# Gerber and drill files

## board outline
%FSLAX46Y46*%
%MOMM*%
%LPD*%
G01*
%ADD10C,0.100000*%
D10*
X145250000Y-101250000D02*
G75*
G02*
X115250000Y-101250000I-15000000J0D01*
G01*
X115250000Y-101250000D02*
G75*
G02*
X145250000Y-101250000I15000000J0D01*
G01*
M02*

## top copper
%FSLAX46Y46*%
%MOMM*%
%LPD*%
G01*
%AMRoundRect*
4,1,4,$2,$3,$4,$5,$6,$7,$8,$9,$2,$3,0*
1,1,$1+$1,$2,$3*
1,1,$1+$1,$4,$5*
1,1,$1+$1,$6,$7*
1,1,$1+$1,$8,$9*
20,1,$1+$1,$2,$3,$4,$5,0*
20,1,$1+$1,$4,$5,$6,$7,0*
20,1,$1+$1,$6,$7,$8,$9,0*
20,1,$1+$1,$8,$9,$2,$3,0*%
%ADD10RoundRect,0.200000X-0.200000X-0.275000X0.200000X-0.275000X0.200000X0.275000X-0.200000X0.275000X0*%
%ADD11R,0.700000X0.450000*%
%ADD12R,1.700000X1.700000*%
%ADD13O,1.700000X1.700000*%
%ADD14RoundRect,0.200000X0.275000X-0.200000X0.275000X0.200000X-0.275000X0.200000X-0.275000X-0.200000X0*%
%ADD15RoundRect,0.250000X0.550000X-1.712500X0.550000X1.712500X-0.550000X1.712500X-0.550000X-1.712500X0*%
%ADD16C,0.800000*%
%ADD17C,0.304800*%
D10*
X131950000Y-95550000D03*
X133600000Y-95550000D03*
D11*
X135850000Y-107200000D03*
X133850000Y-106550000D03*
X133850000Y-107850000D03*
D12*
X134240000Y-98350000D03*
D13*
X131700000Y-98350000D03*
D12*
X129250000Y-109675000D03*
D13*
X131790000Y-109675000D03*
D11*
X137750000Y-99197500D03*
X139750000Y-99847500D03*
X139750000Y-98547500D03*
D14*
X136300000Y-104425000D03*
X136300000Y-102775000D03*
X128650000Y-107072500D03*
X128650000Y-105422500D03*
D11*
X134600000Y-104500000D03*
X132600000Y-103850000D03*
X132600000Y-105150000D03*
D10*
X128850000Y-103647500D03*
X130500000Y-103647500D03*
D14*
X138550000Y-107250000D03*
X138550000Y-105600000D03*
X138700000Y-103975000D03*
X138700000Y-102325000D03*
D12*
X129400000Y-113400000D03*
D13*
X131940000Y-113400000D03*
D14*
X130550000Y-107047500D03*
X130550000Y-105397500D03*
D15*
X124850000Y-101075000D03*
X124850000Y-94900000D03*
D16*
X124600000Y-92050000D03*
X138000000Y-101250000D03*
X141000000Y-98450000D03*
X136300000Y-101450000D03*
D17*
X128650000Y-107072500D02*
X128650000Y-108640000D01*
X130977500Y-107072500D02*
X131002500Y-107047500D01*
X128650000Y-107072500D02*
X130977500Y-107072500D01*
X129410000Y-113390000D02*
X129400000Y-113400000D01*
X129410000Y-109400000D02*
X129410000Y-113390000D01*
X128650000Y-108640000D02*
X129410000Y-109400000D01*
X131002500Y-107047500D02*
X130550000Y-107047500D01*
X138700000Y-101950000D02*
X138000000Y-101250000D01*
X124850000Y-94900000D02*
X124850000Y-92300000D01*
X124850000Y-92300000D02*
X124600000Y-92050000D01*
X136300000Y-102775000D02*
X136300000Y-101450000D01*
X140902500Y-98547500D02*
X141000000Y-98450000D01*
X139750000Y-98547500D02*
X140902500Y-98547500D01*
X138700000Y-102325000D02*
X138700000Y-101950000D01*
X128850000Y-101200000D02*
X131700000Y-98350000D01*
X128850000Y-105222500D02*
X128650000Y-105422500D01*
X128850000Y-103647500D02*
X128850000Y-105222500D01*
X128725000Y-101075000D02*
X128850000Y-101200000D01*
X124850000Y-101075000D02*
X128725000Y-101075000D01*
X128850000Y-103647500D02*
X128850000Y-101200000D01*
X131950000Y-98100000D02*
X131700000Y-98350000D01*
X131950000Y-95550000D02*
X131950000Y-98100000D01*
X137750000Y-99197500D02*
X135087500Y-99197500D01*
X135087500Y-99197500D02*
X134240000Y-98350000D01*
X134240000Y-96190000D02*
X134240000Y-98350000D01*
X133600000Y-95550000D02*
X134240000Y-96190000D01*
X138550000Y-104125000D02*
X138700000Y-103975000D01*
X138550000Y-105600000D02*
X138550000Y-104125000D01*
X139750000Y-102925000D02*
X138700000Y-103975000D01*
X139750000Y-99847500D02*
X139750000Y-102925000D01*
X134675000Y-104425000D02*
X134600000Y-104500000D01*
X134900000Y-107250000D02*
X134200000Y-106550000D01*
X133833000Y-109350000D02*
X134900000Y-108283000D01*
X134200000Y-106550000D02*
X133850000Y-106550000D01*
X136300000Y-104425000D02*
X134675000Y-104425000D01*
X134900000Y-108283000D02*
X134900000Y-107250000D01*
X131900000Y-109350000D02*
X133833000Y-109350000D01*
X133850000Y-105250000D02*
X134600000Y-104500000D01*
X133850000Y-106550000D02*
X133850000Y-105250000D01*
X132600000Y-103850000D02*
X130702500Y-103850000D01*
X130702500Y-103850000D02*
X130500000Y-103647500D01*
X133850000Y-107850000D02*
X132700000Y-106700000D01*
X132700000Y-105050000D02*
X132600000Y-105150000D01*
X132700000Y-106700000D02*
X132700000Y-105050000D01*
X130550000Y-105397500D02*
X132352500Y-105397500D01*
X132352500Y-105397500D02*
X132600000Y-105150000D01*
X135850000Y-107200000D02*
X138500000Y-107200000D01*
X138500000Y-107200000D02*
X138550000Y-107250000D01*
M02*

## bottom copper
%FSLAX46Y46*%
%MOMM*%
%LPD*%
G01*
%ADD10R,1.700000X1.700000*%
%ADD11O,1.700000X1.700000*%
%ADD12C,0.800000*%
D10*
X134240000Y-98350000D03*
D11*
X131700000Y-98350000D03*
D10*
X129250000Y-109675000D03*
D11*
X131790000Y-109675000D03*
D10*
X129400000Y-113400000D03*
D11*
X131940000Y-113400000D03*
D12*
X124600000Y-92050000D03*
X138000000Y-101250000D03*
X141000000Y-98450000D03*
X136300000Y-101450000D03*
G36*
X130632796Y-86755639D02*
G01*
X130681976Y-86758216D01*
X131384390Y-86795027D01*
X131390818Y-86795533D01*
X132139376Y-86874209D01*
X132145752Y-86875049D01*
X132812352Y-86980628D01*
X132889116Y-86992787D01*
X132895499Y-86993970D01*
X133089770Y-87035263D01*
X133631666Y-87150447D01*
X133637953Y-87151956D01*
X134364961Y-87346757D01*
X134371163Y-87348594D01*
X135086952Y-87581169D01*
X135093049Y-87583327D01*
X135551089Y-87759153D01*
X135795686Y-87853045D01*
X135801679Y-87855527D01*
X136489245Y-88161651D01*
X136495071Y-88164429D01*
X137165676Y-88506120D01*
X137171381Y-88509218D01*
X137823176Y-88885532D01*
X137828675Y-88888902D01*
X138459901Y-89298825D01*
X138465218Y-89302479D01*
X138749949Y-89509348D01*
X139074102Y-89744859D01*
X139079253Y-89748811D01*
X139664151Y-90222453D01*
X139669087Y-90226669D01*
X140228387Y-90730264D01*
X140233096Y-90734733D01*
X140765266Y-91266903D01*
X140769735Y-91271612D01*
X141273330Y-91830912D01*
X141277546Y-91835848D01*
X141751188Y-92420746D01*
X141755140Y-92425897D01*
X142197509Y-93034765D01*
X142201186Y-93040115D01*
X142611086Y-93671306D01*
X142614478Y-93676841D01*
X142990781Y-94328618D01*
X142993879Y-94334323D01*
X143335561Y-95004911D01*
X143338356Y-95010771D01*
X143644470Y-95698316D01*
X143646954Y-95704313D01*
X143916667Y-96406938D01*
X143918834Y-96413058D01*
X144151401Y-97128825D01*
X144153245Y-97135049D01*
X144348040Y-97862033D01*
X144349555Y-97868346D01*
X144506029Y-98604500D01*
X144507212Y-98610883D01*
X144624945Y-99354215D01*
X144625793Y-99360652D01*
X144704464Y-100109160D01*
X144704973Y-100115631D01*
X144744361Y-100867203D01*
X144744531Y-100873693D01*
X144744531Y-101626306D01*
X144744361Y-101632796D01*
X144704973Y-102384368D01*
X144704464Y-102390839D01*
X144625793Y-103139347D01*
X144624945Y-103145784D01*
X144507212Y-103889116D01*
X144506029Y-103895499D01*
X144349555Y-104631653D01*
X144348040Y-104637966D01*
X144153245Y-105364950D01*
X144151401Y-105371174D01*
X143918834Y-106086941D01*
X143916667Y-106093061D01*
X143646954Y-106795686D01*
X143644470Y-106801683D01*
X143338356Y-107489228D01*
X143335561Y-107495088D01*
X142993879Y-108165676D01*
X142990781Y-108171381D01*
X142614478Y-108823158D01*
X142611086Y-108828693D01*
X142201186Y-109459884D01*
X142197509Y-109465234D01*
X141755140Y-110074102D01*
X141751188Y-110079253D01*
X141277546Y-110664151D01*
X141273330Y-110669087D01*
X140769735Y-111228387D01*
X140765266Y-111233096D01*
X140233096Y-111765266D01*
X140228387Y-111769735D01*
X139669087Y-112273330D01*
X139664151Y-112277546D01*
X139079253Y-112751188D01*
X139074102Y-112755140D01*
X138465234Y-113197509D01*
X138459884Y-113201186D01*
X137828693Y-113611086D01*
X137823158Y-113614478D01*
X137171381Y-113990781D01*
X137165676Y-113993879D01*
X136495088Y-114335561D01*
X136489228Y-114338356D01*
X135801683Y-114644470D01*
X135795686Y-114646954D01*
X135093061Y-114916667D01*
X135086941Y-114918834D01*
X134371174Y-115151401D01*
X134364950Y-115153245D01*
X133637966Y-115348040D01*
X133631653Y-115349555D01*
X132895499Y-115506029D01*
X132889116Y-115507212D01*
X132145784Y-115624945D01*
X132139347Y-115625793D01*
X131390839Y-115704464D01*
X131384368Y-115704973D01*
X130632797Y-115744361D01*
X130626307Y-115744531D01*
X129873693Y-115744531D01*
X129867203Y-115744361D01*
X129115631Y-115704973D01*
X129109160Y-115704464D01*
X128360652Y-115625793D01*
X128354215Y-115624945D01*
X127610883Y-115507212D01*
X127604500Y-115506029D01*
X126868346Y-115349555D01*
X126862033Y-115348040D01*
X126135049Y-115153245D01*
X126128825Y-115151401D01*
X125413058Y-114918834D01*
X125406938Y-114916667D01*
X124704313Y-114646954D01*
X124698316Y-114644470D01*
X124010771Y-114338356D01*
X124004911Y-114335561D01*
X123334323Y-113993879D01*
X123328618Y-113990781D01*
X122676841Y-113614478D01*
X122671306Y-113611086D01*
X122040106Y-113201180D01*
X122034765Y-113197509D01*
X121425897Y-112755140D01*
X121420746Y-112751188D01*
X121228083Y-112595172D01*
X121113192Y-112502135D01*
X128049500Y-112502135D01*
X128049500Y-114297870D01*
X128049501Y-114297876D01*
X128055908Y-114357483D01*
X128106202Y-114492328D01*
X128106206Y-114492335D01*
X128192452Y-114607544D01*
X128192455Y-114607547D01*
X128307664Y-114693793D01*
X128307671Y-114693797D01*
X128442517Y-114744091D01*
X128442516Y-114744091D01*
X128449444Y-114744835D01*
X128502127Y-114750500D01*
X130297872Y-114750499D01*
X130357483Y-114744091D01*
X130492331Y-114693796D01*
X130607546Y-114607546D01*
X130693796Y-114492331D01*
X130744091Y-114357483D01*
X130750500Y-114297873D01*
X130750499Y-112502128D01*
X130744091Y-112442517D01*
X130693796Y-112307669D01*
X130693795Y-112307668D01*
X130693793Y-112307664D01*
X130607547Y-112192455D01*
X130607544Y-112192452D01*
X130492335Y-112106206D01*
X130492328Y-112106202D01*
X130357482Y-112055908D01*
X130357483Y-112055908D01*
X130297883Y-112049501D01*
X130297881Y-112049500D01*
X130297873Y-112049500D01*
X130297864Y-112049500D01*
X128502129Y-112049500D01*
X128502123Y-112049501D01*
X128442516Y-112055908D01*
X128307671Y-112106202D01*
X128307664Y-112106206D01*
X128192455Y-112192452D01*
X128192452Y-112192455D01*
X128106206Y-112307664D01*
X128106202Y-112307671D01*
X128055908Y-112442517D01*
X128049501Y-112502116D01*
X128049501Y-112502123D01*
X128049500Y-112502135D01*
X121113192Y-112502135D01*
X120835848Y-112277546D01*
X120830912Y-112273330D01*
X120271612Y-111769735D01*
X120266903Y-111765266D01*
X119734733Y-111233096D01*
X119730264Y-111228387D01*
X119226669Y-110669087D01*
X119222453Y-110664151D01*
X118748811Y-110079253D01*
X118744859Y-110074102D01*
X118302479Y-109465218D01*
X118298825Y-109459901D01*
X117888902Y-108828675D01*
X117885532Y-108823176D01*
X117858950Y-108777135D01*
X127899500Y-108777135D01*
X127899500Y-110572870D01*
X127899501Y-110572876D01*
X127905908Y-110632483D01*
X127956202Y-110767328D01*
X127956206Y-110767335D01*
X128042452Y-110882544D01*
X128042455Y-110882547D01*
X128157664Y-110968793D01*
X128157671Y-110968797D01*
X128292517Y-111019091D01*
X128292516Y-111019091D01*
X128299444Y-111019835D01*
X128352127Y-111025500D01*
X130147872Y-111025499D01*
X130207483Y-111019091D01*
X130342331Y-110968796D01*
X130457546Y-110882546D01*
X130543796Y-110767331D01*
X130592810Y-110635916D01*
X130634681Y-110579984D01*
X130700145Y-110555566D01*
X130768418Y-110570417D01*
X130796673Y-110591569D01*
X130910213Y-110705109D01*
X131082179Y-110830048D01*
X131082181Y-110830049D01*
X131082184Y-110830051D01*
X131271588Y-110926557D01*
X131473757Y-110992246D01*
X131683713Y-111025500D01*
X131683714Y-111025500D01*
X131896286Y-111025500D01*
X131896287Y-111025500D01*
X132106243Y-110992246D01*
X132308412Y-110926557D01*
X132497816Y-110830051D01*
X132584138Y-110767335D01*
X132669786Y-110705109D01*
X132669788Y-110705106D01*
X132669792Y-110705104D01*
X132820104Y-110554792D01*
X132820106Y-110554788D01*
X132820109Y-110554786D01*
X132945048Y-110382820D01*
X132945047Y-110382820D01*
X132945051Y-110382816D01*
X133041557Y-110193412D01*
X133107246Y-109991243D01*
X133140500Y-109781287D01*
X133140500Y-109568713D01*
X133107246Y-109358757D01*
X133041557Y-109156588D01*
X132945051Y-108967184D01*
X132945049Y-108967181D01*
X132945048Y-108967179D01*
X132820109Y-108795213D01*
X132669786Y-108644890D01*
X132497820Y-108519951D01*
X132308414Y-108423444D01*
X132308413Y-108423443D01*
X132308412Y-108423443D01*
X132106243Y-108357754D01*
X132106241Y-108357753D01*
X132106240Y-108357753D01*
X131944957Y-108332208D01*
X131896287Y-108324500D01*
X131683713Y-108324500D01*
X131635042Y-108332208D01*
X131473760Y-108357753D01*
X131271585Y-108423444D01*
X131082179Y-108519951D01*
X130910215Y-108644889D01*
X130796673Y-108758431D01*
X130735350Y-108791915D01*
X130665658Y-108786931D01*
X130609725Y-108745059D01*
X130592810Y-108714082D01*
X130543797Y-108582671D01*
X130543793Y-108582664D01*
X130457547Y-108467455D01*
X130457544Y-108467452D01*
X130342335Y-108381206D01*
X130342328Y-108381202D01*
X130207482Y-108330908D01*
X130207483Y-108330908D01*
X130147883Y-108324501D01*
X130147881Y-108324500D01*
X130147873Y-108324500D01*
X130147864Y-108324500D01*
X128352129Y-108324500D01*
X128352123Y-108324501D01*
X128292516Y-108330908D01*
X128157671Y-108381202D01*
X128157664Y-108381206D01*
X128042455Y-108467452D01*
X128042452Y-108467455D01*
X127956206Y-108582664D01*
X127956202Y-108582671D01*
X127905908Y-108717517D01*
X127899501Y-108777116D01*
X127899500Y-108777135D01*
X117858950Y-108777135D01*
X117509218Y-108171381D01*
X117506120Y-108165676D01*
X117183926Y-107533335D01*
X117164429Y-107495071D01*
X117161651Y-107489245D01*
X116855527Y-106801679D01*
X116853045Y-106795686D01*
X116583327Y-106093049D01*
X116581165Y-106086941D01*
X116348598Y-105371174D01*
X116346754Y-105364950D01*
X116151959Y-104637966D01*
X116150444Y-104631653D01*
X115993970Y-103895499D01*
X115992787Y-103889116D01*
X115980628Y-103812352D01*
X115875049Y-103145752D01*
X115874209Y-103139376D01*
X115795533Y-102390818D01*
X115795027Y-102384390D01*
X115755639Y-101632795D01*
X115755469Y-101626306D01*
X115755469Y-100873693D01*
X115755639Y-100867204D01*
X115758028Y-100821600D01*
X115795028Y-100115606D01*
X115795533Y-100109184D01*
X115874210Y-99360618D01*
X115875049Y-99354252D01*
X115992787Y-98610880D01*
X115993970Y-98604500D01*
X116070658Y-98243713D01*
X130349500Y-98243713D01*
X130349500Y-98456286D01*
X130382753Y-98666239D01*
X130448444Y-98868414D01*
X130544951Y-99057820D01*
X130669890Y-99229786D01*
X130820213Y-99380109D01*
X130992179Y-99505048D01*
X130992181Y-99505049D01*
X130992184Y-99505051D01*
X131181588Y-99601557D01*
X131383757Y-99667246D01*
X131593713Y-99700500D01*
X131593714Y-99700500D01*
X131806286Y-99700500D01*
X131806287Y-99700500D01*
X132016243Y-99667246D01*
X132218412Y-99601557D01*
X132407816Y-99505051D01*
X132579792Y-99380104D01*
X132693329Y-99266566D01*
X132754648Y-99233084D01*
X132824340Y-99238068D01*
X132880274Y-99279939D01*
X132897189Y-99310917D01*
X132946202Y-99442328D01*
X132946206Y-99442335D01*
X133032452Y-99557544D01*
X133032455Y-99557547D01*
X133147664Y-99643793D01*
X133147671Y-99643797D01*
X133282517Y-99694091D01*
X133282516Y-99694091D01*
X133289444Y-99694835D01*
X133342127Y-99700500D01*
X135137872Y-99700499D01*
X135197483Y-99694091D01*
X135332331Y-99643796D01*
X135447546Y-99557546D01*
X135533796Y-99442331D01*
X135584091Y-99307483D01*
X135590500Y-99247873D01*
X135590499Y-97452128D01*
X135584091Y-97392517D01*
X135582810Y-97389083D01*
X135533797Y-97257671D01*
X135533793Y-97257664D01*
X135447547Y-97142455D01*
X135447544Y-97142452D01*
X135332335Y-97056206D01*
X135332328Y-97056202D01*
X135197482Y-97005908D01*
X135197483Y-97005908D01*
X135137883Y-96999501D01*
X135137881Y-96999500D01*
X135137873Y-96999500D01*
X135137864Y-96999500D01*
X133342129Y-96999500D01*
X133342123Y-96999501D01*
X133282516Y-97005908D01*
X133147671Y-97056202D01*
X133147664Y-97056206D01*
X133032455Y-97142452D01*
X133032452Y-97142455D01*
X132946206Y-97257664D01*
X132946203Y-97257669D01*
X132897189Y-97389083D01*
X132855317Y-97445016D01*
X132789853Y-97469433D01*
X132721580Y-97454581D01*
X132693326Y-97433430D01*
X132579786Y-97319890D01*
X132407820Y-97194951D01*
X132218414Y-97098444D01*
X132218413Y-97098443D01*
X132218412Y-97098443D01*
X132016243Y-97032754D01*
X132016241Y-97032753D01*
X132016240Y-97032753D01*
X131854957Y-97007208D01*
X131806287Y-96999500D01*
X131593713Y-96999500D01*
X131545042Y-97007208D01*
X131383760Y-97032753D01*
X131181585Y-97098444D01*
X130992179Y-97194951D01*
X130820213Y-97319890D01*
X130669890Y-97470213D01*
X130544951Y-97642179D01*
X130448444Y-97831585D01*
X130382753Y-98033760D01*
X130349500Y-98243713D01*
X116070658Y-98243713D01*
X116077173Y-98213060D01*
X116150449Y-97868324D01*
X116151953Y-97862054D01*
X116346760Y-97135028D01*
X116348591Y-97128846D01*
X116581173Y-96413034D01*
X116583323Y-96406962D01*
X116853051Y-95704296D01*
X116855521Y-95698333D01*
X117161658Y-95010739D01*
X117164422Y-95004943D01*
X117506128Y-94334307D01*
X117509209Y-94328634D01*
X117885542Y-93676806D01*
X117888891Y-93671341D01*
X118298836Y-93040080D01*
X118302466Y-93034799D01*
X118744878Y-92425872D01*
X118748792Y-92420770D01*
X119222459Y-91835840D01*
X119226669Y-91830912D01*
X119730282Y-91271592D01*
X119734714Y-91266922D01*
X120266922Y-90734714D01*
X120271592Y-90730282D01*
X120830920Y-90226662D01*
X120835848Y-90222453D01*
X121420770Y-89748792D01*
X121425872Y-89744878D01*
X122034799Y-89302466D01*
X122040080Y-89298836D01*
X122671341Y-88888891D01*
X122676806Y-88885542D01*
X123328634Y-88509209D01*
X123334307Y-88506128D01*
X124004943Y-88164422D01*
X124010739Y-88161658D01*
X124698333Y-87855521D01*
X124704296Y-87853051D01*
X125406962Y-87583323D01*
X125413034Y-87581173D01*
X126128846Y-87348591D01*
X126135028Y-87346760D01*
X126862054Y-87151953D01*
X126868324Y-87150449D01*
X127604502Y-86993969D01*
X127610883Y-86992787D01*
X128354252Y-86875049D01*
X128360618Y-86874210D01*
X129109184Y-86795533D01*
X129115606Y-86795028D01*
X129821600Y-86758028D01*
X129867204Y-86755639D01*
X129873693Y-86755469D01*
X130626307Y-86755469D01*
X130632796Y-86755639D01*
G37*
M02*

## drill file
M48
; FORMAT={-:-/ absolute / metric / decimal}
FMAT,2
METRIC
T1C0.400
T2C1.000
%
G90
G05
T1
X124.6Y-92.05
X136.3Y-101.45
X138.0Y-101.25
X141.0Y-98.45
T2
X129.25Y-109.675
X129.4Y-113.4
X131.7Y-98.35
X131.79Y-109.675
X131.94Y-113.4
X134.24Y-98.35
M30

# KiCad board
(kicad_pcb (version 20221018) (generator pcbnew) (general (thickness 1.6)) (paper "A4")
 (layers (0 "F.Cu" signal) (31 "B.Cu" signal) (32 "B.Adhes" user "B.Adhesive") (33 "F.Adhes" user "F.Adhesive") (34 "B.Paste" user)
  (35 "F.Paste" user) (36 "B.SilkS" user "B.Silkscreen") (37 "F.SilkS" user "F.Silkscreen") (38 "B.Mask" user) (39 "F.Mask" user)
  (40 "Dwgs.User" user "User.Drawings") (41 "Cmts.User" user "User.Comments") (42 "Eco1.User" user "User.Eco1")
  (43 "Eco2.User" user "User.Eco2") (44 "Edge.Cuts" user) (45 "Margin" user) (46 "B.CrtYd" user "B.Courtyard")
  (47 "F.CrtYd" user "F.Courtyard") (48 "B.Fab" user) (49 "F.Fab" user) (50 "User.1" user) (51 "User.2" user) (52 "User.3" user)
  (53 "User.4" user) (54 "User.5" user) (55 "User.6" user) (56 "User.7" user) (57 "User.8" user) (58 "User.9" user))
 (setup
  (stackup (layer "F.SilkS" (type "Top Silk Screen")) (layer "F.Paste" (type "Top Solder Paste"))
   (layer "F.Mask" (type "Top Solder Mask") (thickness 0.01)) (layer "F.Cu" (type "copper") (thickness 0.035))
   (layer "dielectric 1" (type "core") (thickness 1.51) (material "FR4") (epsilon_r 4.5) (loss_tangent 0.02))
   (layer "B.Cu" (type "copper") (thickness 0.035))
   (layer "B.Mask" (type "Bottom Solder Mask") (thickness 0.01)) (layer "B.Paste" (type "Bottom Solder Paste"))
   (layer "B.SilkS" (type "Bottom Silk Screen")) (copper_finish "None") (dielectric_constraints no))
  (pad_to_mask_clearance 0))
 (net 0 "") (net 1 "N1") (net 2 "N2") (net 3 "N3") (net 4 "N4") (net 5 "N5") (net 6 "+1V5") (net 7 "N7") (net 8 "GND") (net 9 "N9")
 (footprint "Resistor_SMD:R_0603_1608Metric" (layer "F.Cu") (at 132.775 95.55)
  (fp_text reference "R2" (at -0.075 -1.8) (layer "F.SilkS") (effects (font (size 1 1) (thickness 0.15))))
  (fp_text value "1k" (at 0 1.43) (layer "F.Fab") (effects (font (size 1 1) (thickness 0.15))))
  (pad "1" smd roundrect (at -0.825 0) (size 0.8 0.95) (layers "F.Cu" "F.Paste" "F.Mask") (roundrect_rratio 0.25) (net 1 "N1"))
  (pad "2" smd roundrect (at 0.825 0) (size 0.8 0.95) (layers "F.Cu" "F.Paste" "F.Mask") (roundrect_rratio 0.25) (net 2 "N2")))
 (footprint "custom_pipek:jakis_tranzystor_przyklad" (layer "F.Cu") (at 134.55 105.92)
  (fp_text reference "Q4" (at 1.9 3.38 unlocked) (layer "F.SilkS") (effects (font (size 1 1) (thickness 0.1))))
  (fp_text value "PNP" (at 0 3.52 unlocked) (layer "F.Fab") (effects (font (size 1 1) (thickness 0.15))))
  (pad "1" smd rect (at 1.3 1.28 270) (size 0.45 0.7) (layers "F.Cu" "F.Paste" "F.Mask") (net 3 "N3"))
  (pad "2" smd rect (at -0.7 0.63 270) (size 0.45 0.7) (layers "F.Cu" "F.Paste" "F.Mask") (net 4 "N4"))
  (pad "3" smd rect (at -0.7 1.93 270) (size 0.45 0.7) (layers "F.Cu" "F.Paste" "F.Mask") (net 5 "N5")))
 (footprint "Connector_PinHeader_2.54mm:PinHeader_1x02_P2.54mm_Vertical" (layer "F.Cu") (at 134.24 98.35 -90)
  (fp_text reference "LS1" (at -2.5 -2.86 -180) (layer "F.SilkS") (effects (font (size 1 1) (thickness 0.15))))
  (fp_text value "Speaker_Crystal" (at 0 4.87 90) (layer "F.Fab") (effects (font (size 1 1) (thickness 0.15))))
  (pad "1" thru_hole rect (at 0 0 270) (size 1.7 1.7) (drill 1) (layers "*.Cu" "*.Mask") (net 2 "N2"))
  (pad "2" thru_hole oval (at 0 2.54 270) (size 1.7 1.7) (drill 1) (layers "*.Cu" "*.Mask") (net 1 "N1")))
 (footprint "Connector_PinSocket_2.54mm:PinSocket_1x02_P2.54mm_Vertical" (layer "F.Cu") (at 129.25 109.675 90)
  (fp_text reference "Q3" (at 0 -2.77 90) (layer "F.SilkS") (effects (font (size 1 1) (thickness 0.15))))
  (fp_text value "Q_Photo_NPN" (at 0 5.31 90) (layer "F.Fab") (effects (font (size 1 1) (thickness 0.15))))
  (pad "1" thru_hole rect (at 0 0 90) (size 1.7 1.7) (drill 1) (layers "*.Cu" "*.Mask") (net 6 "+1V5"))
  (pad "2" thru_hole oval (at 0 2.54 90) (size 1.7 1.7) (drill 1) (layers "*.Cu" "*.Mask") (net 4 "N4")))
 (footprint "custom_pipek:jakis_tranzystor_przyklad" (layer "F.Cu") (at 139.05 100.4775 180)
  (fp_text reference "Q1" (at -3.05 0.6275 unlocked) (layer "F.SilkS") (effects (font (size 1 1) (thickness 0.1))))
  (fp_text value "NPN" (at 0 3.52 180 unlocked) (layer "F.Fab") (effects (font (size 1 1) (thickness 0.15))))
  (pad "1" smd rect (at 1.3 1.28 90) (size 0.45 0.7) (layers "F.Cu" "F.Paste" "F.Mask") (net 2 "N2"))
  (pad "2" smd rect (at -0.7 0.63 90) (size 0.45 0.7) (layers "F.Cu" "F.Paste" "F.Mask") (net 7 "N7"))
  (pad "3" smd rect (at -0.7 1.93 90) (size 0.45 0.7) (layers "F.Cu" "F.Paste" "F.Mask") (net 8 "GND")))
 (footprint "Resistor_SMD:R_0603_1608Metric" (layer "F.Cu") (at 136.3 103.6 90)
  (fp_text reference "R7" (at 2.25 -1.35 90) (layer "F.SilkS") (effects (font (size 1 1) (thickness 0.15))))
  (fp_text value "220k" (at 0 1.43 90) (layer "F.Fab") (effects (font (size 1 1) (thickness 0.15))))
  (pad "1" smd roundrect (at -0.825 0 90) (size 0.8 0.95) (layers "F.Cu" "F.Paste" "F.Mask") (roundrect_rratio 0.25) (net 4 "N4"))
  (pad "2" smd roundrect (at 0.825 0 90) (size 0.8 0.95) (layers "F.Cu" "F.Paste" "F.Mask") (roundrect_rratio 0.25) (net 8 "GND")))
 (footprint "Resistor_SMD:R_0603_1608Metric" (layer "F.Cu") (at 128.65 106.2475 90)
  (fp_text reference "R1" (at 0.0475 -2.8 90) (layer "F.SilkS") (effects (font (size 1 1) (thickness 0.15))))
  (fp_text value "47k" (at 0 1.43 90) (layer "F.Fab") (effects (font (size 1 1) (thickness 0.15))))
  (pad "1" smd roundrect (at -0.825 0 90) (size 0.8 0.95) (layers "F.Cu" "F.Paste" "F.Mask") (roundrect_rratio 0.25) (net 6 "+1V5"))
  (pad "2" smd roundrect (at 0.825 0 90) (size 0.8 0.95) (layers "F.Cu" "F.Paste" "F.Mask") (roundrect_rratio 0.25) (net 1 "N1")))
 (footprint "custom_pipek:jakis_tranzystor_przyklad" (layer "F.Cu") (at 133.3 103.22)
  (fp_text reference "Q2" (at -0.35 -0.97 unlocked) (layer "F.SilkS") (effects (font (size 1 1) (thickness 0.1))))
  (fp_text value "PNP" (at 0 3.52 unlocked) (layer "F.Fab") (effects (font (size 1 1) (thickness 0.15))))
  (pad "1" smd rect (at 1.3 1.28 270) (size 0.45 0.7) (layers "F.Cu" "F.Paste" "F.Mask") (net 4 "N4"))
  (pad "2" smd rect (at -0.7 0.63 270) (size 0.45 0.7) (layers "F.Cu" "F.Paste" "F.Mask") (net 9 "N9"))
  (pad "3" smd rect (at -0.7 1.93 270) (size 0.45 0.7) (layers "F.Cu" "F.Paste" "F.Mask") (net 5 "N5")))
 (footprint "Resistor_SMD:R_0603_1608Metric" (layer "F.Cu") (at 129.675 103.6475)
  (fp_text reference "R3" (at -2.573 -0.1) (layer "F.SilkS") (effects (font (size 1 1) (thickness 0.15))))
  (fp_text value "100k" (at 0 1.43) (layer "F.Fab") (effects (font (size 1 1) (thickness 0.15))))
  (pad "1" smd roundrect (at -0.825 0) (size 0.8 0.95) (layers "F.Cu" "F.Paste" "F.Mask") (roundrect_rratio 0.25) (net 1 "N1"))
  (pad "2" smd roundrect (at 0.825 0) (size 0.8 0.95) (layers "F.Cu" "F.Paste" "F.Mask") (roundrect_rratio 0.25) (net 9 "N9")))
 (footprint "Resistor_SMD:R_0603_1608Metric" (layer "F.Cu") (at 138.55 106.425 90)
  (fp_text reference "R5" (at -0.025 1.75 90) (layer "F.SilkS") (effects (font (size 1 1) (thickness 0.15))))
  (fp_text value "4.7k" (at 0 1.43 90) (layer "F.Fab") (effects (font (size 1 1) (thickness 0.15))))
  (pad "1" smd roundrect (at -0.825 0 90) (size 0.8 0.95) (layers "F.Cu" "F.Paste" "F.Mask") (roundrect_rratio 0.25) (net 3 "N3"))
  (pad "2" smd roundrect (at 0.825 0 90) (size 0.8 0.95) (layers "F.Cu" "F.Paste" "F.Mask") (roundrect_rratio 0.25) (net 7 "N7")))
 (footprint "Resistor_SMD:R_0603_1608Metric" (layer "F.Cu") (at 138.7 103.15 90)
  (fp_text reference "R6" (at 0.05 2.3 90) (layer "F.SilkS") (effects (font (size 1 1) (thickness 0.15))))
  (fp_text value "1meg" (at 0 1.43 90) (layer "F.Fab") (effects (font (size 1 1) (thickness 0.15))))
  (pad "1" smd roundrect (at -0.825 0 90) (size 0.8 0.95) (layers "F.Cu" "F.Paste" "F.Mask") (roundrect_rratio 0.25) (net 7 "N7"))
  (pad "2" smd roundrect (at 0.825 0 90) (size 0.8 0.95) (layers "F.Cu" "F.Paste" "F.Mask") (roundrect_rratio 0.25) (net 8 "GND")))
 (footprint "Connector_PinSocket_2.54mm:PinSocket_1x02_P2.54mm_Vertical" (layer "F.Cu") (at 129.4 113.4 90)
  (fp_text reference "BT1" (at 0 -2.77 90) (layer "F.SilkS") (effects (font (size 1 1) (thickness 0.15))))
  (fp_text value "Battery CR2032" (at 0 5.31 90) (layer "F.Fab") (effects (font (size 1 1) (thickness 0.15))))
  (pad "1" thru_hole rect (at 0 0 90) (size 1.7 1.7) (drill 1) (layers "*.Cu" "*.Mask") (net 6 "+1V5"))
  (pad "2" thru_hole oval (at 0 2.54 90) (size 1.7 1.7) (drill 1) (layers "*.Cu" "*.Mask") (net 8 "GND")))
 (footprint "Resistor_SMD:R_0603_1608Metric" (layer "F.Cu") (at 130.55 106.2225 90)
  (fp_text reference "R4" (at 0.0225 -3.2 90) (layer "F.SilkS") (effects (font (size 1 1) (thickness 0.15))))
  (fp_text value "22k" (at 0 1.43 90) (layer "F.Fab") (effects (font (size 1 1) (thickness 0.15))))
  (pad "1" smd roundrect (at -0.825 0 90) (size 0.8 0.95) (layers "F.Cu" "F.Paste" "F.Mask") (roundrect_rratio 0.25) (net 6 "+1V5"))
  (pad "2" smd roundrect (at 0.825 0 90) (size 0.8 0.95) (layers "F.Cu" "F.Paste" "F.Mask") (roundrect_rratio 0.25) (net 5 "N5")))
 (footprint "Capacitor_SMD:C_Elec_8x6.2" (layer "F.Cu") (at 124.85 97.9875 90)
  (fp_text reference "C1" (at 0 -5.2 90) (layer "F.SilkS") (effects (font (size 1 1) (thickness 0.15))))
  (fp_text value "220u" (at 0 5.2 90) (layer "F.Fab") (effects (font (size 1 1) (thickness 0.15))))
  (pad "1" smd roundrect (at -3.0875 0 90) (size 3.925 1.6) (layers "F.Cu" "F.Paste" "F.Mask") (roundrect_rratio 0.15625) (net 1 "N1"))
  (pad "2" smd roundrect (at 3.0875 0 90) (size 3.925 1.6) (layers "F.Cu" "F.Paste" "F.Mask") (roundrect_rratio 0.15625) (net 8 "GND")))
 (gr_circle locked (center 130.25 101.25) (end 145.25 101.25) (stroke (width 0.1) (type default)) (fill none) (layer "Edge.Cuts"))
 (segment (start 128.65 107.0725) (end 128.65 108.64) (width 0.3048) (layer "F.Cu") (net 6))
 (segment (start 130.9775 107.0725) (end 131.0025 107.0475) (width 0.3048) (layer "F.Cu") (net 6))
 (segment (start 128.65 107.0725) (end 130.9775 107.0725) (width 0.3048) (layer "F.Cu") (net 6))
 (segment (start 129.41 113.39) (end 129.4 113.4) (width 0.3048) (layer "F.Cu") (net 6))
 (segment (start 129.41 109.4) (end 129.41 113.39) (width 0.3048) (layer "F.Cu") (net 6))
 (segment (start 128.65 108.64) (end 129.41 109.4) (width 0.3048) (layer "F.Cu") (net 6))
 (segment (start 131.0025 107.0475) (end 130.55 107.0475) (width 0.3048) (layer "F.Cu") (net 6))
 (segment (start 138.7 101.95) (end 138 101.25) (width 0.3048) (layer "F.Cu") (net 8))
 (segment (start 124.85 94.9) (end 124.85 92.3) (width 0.3048) (layer "F.Cu") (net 8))
 (segment (start 124.85 92.3) (end 124.6 92.05) (width 0.3048) (layer "F.Cu") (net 8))
 (segment (start 136.3 102.775) (end 136.3 101.45) (width 0.3048) (layer "F.Cu") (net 8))
 (segment (start 140.9025 98.5475) (end 141 98.45) (width 0.3048) (layer "F.Cu") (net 8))
 (segment (start 139.75 98.5475) (end 140.9025 98.5475) (width 0.3048) (layer "F.Cu") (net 8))
 (segment (start 138.7 102.325) (end 138.7 101.95) (width 0.3048) (layer "F.Cu") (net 8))
 (via (at 124.6 92.05) (size 0.8) (drill 0.4) (layers "F.Cu" "B.Cu") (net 8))
 (via (at 138 101.25) (size 0.8) (drill 0.4) (layers "F.Cu" "B.Cu") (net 8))
 (via (at 141 98.45) (size 0.8) (drill 0.4) (layers "F.Cu" "B.Cu") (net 8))
 (via (at 136.3 101.45) (size 0.8) (drill 0.4) (layers "F.Cu" "B.Cu") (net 8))
 (segment (start 128.85 101.2) (end 131.7 98.35) (width 0.3048) (layer "F.Cu") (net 1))
 (segment (start 128.85 105.2225) (end 128.65 105.4225) (width 0.3048) (layer "F.Cu") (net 1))
 (segment (start 128.85 103.6475) (end 128.85 105.2225) (width 0.3048) (layer "F.Cu") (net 1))
 (segment (start 128.725 101.075) (end 128.85 101.2) (width 0.3048) (layer "F.Cu") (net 1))
 (segment (start 124.85 101.075) (end 128.725 101.075) (width 0.3048) (layer "F.Cu") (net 1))
 (segment (start 128.85 103.6475) (end 128.85 101.2) (width 0.3048) (layer "F.Cu") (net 1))
 (segment (start 131.95 98.1) (end 131.7 98.35) (width 0.3048) (layer "F.Cu") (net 1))
 (segment (start 131.95 95.55) (end 131.95 98.1) (width 0.3048) (layer "F.Cu") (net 1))
 (segment (start 137.75 99.1975) (end 135.0875 99.1975) (width 0.3048) (layer "F.Cu") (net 2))
 (segment (start 135.0875 99.1975) (end 134.24 98.35) (width 0.3048) (layer "F.Cu") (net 2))
 (segment (start 134.24 96.19) (end 134.24 98.35) (width 0.3048) (layer "F.Cu") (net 2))
 (segment (start 133.6 95.55) (end 134.24 96.19) (width 0.3048) (layer "F.Cu") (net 2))
 (segment (start 138.55 104.125) (end 138.7 103.975) (width 0.3048) (layer "F.Cu") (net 7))
 (segment (start 138.55 105.6) (end 138.55 104.125) (width 0.3048) (layer "F.Cu") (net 7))
 (segment (start 139.75 102.925) (end 138.7 103.975) (width 0.3048) (layer "F.Cu") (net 7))
 (segment (start 139.75 99.8475) (end 139.75 102.925) (width 0.3048) (layer "F.Cu") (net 7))
 (segment (start 134.675 104.425) (end 134.6 104.5) (width 0.3048) (layer "F.Cu") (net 4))
 (segment (start 134.9 107.25) (end 134.2 106.55) (width 0.3048) (layer "F.Cu") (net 4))
 (segment (start 133.833 109.35) (end 134.9 108.283) (width 0.3048) (layer "F.Cu") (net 4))
 (segment (start 134.2 106.55) (end 133.85 106.55) (width 0.3048) (layer "F.Cu") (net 4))
 (segment (start 136.3 104.425) (end 134.675 104.425) (width 0.3048) (layer "F.Cu") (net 4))
 (segment (start 134.9 108.283) (end 134.9 107.25) (width 0.3048) (layer "F.Cu") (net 4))
 (segment (start 131.9 109.35) (end 133.833 109.35) (width 0.3048) (layer "F.Cu") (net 4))
 (segment (start 133.85 105.25) (end 134.6 104.5) (width 0.3048) (layer "F.Cu") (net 4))
 (segment (start 133.85 106.55) (end 133.85 105.25) (width 0.3048) (layer "F.Cu") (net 4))
 (segment (start 132.6 103.85) (end 130.7025 103.85) (width 0.3048) (layer "F.Cu") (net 9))
 (segment (start 130.7025 103.85) (end 130.5 103.6475) (width 0.3048) (layer "F.Cu") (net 9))
 (segment (start 133.85 107.85) (end 132.7 106.7) (width 0.3048) (layer "F.Cu") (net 5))
 (segment (start 132.7 105.05) (end 132.6 105.15) (width 0.3048) (layer "F.Cu") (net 5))
 (segment (start 132.7 106.7) (end 132.7 105.05) (width 0.3048) (layer "F.Cu") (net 5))
 (segment (start 130.55 105.3975) (end 132.3525 105.3975) (width 0.3048) (layer "F.Cu") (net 5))
 (segment (start 132.3525 105.3975) (end 132.6 105.15) (width 0.3048) (layer "F.Cu") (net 5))
 (segment (start 135.85 107.2) (end 138.5 107.2) (width 0.3048) (layer "F.Cu") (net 3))
 (segment (start 138.5 107.2) (end 138.55 107.25) (width 0.3048) (layer "F.Cu") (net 3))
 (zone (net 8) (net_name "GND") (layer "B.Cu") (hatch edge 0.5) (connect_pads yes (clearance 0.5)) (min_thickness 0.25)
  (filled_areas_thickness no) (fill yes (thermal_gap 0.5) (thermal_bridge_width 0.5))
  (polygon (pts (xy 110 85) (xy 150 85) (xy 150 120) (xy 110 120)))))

